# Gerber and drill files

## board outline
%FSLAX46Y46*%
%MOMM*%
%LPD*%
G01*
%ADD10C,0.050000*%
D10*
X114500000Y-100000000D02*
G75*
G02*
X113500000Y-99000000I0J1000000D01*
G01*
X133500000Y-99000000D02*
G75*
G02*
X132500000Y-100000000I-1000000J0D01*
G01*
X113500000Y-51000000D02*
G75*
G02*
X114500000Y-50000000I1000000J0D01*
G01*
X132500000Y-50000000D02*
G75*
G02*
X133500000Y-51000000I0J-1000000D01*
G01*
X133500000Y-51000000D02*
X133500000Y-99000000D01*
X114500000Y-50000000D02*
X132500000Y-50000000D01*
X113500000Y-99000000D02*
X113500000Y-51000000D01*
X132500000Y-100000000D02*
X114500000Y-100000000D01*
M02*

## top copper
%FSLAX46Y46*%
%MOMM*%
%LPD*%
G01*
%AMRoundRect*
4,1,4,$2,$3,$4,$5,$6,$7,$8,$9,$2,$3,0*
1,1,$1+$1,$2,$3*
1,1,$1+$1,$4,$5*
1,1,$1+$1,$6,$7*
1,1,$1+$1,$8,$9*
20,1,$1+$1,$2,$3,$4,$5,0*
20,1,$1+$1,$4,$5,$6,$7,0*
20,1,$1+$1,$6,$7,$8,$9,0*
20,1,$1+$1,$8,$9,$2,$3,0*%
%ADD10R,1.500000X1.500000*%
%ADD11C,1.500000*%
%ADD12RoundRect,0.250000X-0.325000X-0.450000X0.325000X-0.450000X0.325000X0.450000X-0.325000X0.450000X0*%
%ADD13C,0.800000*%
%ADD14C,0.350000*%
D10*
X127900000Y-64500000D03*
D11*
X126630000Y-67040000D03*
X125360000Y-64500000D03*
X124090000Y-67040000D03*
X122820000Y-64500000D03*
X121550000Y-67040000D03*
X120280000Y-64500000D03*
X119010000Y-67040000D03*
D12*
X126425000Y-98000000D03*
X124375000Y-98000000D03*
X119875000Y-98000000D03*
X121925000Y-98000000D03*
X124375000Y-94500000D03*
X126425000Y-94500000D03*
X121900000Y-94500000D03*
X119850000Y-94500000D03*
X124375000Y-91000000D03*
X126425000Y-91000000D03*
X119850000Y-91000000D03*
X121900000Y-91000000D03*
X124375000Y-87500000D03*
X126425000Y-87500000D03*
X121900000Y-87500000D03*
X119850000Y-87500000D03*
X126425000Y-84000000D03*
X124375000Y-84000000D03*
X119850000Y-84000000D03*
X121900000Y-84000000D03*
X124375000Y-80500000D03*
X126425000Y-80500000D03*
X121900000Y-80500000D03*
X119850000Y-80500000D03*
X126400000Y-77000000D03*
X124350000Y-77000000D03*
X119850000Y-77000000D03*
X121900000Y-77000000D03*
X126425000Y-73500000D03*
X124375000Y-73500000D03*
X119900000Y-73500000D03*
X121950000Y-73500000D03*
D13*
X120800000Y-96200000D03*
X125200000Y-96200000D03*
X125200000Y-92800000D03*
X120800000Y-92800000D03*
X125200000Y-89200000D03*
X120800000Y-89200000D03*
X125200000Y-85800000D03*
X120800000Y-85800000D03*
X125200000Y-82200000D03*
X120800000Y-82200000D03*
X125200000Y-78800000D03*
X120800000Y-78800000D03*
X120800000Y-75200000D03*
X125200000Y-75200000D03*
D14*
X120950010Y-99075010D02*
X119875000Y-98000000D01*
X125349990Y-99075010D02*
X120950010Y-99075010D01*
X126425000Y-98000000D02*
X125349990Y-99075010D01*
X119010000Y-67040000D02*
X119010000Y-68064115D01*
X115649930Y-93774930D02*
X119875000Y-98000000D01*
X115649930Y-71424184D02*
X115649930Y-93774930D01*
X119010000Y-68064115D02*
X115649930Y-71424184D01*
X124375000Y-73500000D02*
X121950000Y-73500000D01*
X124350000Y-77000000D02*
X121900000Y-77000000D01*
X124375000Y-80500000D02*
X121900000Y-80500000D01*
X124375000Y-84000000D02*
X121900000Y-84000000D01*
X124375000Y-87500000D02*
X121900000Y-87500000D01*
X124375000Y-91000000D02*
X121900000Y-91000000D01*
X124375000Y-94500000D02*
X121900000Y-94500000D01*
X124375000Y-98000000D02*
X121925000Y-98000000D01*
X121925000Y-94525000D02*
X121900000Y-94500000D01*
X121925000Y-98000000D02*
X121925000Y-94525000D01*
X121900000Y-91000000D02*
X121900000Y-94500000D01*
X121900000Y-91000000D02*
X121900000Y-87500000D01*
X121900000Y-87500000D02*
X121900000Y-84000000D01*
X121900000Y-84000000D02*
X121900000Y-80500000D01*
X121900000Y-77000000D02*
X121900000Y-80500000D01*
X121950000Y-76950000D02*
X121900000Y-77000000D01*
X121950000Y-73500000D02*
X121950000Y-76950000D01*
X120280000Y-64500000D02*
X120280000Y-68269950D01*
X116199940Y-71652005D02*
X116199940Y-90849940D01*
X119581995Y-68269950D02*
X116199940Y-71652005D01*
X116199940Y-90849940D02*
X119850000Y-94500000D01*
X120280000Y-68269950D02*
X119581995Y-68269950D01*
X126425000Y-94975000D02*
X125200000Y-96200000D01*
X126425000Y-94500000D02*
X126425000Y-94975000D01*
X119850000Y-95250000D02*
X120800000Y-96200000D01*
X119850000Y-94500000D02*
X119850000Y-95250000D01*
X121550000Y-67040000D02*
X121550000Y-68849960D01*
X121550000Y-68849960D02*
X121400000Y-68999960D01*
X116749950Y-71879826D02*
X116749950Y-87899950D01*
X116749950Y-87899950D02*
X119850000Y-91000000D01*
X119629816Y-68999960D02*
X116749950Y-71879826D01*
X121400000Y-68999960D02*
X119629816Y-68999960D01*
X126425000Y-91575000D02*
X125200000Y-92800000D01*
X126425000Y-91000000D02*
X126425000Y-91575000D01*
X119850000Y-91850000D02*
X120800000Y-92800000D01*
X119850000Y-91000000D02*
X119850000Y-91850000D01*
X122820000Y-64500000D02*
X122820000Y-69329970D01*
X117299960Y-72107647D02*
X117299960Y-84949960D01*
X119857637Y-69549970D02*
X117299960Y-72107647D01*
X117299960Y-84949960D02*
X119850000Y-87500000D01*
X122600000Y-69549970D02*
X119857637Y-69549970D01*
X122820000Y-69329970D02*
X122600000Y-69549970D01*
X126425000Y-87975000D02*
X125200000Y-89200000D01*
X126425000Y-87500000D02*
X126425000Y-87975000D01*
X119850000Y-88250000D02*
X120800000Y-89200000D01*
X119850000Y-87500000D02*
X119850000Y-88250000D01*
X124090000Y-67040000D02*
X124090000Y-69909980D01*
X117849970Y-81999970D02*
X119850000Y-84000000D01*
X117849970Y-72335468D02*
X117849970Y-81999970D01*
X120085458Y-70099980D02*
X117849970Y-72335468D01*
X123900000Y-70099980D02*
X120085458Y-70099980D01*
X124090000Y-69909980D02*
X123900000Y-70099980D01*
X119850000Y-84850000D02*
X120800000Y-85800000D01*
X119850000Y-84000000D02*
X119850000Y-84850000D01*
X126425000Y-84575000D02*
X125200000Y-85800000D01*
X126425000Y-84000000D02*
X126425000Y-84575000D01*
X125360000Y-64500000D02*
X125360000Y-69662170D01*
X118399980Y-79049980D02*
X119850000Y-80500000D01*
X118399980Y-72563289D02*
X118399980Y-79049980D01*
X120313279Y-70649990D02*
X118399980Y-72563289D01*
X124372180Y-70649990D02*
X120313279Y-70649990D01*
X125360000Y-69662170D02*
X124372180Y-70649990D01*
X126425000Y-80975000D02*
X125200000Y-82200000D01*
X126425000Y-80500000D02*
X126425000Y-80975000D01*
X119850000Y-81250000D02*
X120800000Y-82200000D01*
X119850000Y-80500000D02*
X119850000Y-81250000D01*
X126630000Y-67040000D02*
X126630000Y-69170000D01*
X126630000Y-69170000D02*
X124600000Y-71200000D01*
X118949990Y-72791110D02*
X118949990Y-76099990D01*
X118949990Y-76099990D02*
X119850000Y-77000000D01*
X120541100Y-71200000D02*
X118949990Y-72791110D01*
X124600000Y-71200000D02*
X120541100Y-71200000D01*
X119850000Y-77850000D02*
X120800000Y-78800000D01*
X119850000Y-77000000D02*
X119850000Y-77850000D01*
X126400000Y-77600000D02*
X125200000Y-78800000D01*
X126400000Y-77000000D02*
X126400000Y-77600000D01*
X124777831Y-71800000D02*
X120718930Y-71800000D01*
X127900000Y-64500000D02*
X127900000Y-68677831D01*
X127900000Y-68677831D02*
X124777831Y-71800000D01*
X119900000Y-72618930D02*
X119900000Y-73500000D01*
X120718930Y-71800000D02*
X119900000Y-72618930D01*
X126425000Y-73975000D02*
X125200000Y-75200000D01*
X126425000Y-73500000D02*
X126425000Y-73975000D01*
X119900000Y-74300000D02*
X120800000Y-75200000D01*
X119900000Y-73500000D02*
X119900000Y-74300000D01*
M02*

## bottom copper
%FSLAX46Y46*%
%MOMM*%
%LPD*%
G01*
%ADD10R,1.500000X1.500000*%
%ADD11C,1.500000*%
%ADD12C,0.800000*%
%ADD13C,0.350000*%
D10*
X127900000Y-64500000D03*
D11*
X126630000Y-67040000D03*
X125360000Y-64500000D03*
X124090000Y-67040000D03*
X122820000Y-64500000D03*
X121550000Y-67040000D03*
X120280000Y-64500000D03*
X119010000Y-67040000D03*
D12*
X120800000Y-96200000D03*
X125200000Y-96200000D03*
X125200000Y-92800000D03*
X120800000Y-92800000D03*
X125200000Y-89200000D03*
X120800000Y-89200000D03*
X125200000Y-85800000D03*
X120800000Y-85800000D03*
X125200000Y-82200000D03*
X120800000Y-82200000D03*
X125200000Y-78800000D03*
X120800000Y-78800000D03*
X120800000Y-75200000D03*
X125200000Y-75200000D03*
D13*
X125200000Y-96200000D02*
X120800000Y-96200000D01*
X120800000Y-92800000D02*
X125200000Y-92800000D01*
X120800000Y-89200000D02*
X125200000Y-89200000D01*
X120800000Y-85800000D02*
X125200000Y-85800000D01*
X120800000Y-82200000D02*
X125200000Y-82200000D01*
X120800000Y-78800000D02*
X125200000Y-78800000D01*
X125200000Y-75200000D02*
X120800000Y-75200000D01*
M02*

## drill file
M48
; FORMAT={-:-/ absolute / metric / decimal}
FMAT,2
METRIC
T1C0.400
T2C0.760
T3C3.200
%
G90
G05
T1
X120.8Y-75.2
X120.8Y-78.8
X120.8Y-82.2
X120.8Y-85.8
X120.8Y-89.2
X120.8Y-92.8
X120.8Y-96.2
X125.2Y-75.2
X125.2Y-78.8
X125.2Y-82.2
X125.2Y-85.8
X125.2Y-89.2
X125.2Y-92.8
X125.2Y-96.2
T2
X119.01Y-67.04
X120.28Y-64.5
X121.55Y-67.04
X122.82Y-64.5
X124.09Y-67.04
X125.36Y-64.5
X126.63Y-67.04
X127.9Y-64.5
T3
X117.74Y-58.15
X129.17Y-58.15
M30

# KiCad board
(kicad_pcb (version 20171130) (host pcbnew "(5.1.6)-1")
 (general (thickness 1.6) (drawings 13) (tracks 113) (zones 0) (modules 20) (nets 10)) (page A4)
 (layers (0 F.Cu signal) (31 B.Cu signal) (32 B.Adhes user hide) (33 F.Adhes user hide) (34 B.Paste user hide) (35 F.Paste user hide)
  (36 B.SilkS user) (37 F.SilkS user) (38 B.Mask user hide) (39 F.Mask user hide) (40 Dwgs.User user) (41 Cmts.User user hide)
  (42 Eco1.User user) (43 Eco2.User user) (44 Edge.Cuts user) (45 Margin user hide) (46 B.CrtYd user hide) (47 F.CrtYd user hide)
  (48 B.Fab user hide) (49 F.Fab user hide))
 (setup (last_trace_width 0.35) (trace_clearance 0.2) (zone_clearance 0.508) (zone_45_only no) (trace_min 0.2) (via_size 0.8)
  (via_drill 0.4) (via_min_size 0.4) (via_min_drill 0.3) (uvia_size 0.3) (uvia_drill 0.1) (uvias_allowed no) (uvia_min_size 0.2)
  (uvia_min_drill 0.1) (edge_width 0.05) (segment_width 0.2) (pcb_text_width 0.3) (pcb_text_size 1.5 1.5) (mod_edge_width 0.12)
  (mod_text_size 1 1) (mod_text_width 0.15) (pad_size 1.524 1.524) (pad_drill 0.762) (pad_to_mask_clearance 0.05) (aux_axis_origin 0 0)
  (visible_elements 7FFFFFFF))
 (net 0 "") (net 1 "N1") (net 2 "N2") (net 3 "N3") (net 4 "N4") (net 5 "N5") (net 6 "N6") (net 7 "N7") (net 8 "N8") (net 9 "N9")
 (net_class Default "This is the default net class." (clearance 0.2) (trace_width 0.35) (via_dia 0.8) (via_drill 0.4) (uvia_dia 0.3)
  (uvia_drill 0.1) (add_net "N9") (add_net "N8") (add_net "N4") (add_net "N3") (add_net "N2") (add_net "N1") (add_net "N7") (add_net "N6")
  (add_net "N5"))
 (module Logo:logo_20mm (layer B.Cu) (at 123.6 79.8 180)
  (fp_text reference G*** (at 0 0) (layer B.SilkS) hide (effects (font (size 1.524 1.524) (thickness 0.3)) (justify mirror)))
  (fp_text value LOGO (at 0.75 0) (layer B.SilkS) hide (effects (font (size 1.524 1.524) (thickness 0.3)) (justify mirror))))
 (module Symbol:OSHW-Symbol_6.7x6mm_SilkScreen (layer B.Cu) (at 118.1 95.9 180)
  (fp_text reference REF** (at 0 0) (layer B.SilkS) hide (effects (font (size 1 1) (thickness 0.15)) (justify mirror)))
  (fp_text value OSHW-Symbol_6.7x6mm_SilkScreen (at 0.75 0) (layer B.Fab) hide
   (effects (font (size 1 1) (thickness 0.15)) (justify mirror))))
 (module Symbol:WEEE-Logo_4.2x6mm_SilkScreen (layer B.Cu) (at 130.6 95.8 180)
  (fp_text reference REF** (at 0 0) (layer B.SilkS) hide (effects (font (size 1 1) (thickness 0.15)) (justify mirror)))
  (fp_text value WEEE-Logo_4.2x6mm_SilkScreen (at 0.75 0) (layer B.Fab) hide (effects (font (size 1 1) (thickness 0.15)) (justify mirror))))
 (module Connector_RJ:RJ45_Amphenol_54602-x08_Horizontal (layer F.Cu) (at 127.9 64.5 180)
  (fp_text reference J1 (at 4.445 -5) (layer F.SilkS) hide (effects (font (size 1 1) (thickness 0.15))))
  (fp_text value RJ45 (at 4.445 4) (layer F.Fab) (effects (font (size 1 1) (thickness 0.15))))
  (pad "" np_thru_hole circle (at 10.16 6.35 180) (size 3.2 3.2) (drill 3.2) (layers *.Cu *.Mask))
  (pad "" np_thru_hole circle (at -1.27 6.35 180) (size 3.2 3.2) (drill 3.2) (layers *.Cu *.Mask))
  (pad 1 thru_hole rect (at 0 0 180) (size 1.5 1.5) (drill 0.76) (layers *.Cu *.Mask) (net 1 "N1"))
  (pad 2 thru_hole circle (at 1.27 -2.54 180) (size 1.5 1.5) (drill 0.76) (layers *.Cu *.Mask) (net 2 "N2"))
  (pad 3 thru_hole circle (at 2.54 0 180) (size 1.5 1.5) (drill 0.76) (layers *.Cu *.Mask) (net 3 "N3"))
  (pad 4 thru_hole circle (at 3.81 -2.54 180) (size 1.5 1.5) (drill 0.76) (layers *.Cu *.Mask) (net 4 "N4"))
  (pad 5 thru_hole circle (at 5.08 0 180) (size 1.5 1.5) (drill 0.76) (layers *.Cu *.Mask) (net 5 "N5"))
  (pad 6 thru_hole circle (at 6.35 -2.54 180) (size 1.5 1.5) (drill 0.76) (layers *.Cu *.Mask) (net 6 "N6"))
  (pad 7 thru_hole circle (at 7.62 0 180) (size 1.5 1.5) (drill 0.76) (layers *.Cu *.Mask) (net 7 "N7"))
  (pad 8 thru_hole circle (at 8.89 -2.54 180) (size 1.5 1.5) (drill 0.76) (layers *.Cu *.Mask) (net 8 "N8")))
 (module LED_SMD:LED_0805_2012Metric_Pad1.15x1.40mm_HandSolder (layer F.Cu) (at 125.4 98)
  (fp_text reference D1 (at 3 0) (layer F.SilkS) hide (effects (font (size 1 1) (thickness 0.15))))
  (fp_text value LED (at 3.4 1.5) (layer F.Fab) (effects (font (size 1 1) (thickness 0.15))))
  (pad 2 smd roundrect (at 1.025 0) (size 1.15 1.4) (layers F.Cu F.Paste F.Mask) (roundrect_rratio 0.217391) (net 8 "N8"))
  (pad 1 smd roundrect (at -1.025 0) (size 1.15 1.4) (layers F.Cu F.Paste F.Mask) (roundrect_rratio 0.217391) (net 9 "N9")))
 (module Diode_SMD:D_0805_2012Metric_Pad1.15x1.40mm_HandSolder (layer F.Cu) (at 120.9 98)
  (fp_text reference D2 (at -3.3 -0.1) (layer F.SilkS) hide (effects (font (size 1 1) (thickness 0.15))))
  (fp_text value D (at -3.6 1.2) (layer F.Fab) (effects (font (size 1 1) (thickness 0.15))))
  (pad 1 smd roundrect (at -1.025 0) (size 1.15 1.4) (layers F.Cu F.Paste F.Mask) (roundrect_rratio 0.217391) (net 8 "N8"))
  (pad 2 smd roundrect (at 1.025 0) (size 1.15 1.4) (layers F.Cu F.Paste F.Mask) (roundrect_rratio 0.217391) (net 9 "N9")))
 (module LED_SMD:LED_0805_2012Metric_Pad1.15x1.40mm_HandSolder (layer F.Cu) (at 125.4 94.5)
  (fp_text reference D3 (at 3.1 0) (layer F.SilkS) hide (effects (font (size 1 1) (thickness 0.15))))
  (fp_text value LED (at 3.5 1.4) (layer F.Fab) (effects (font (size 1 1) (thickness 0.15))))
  (pad 1 smd roundrect (at -1.025 0) (size 1.15 1.4) (layers F.Cu F.Paste F.Mask) (roundrect_rratio 0.217391) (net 9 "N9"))
  (pad 2 smd roundrect (at 1.025 0) (size 1.15 1.4) (layers F.Cu F.Paste F.Mask) (roundrect_rratio 0.217391) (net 7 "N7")))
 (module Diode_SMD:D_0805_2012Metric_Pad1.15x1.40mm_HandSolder (layer F.Cu) (at 120.875 94.5)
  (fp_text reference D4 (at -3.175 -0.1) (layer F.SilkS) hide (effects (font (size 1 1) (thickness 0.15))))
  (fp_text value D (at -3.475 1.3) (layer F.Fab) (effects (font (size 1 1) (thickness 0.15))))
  (pad 2 smd roundrect (at 1.025 0) (size 1.15 1.4) (layers F.Cu F.Paste F.Mask) (roundrect_rratio 0.217391) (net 9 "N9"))
  (pad 1 smd roundrect (at -1.025 0) (size 1.15 1.4) (layers F.Cu F.Paste F.Mask) (roundrect_rratio 0.217391) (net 7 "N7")))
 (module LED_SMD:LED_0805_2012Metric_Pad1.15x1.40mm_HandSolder (layer F.Cu) (at 125.4 91)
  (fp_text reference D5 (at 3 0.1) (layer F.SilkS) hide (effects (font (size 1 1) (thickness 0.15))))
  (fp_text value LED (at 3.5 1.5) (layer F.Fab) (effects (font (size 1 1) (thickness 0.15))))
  (pad 1 smd roundrect (at -1.025 0) (size 1.15 1.4) (layers F.Cu F.Paste F.Mask) (roundrect_rratio 0.217391) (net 9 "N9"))
  (pad 2 smd roundrect (at 1.025 0) (size 1.15 1.4) (layers F.Cu F.Paste F.Mask) (roundrect_rratio 0.217391) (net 6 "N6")))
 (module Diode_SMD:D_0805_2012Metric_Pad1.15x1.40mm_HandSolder (layer F.Cu) (at 120.875 91)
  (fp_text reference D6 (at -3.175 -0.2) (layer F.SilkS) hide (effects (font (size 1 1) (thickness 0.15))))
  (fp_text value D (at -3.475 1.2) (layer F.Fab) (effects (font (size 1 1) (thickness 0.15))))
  (pad 1 smd roundrect (at -1.025 0) (size 1.15 1.4) (layers F.Cu F.Paste F.Mask) (roundrect_rratio 0.217391) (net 6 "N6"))
  (pad 2 smd roundrect (at 1.025 0) (size 1.15 1.4) (layers F.Cu F.Paste F.Mask) (roundrect_rratio 0.217391) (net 9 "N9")))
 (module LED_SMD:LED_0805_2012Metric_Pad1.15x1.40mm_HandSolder (layer F.Cu) (at 125.4 87.5)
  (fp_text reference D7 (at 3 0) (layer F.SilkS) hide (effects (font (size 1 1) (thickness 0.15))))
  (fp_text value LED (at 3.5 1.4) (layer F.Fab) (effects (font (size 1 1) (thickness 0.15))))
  (pad 1 smd roundrect (at -1.025 0) (size 1.15 1.4) (layers F.Cu F.Paste F.Mask) (roundrect_rratio 0.217391) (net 9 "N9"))
  (pad 2 smd roundrect (at 1.025 0) (size 1.15 1.4) (layers F.Cu F.Paste F.Mask) (roundrect_rratio 0.217391) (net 5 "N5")))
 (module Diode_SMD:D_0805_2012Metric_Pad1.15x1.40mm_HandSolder (layer F.Cu) (at 120.875 87.5)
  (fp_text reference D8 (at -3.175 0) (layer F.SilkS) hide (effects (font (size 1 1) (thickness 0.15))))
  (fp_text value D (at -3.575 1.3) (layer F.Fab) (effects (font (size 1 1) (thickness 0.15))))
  (pad 2 smd roundrect (at 1.025 0) (size 1.15 1.4) (layers F.Cu F.Paste F.Mask) (roundrect_rratio 0.217391) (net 9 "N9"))
  (pad 1 smd roundrect (at -1.025 0) (size 1.15 1.4) (layers F.Cu F.Paste F.Mask) (roundrect_rratio 0.217391) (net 5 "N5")))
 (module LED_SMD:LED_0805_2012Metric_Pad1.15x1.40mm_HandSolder (layer F.Cu) (at 125.4 84)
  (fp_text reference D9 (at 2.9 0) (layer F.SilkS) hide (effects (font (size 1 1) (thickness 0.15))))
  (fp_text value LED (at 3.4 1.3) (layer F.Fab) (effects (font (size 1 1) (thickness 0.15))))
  (pad 2 smd roundrect (at 1.025 0) (size 1.15 1.4) (layers F.Cu F.Paste F.Mask) (roundrect_rratio 0.217391) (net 4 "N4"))
  (pad 1 smd roundrect (at -1.025 0) (size 1.15 1.4) (layers F.Cu F.Paste F.Mask) (roundrect_rratio 0.217391) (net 9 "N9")))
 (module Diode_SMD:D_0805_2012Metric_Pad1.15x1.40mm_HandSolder (layer F.Cu) (at 120.875 84)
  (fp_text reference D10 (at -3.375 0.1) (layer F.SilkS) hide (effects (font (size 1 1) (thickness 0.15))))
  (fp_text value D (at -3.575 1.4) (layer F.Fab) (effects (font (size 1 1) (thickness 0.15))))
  (pad 1 smd roundrect (at -1.025 0) (size 1.15 1.4) (layers F.Cu F.Paste F.Mask) (roundrect_rratio 0.217391) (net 4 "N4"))
  (pad 2 smd roundrect (at 1.025 0) (size 1.15 1.4) (layers F.Cu F.Paste F.Mask) (roundrect_rratio 0.217391) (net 9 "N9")))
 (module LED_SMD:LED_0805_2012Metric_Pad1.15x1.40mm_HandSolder (layer F.Cu) (at 125.4 80.5)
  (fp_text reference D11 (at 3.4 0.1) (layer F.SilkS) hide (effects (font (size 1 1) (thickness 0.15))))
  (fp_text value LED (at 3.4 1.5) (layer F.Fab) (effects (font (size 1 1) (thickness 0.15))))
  (pad 1 smd roundrect (at -1.025 0) (size 1.15 1.4) (layers F.Cu F.Paste F.Mask) (roundrect_rratio 0.217391) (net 9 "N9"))
  (pad 2 smd roundrect (at 1.025 0) (size 1.15 1.4) (layers F.Cu F.Paste F.Mask) (roundrect_rratio 0.217391) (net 3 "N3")))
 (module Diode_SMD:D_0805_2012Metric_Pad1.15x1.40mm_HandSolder (layer F.Cu) (at 120.875 80.5)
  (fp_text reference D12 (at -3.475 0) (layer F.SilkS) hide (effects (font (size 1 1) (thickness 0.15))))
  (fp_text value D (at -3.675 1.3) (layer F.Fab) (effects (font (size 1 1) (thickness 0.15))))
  (pad 2 smd roundrect (at 1.025 0) (size 1.15 1.4) (layers F.Cu F.Paste F.Mask) (roundrect_rratio 0.217391) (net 9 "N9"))
  (pad 1 smd roundrect (at -1.025 0) (size 1.15 1.4) (layers F.Cu F.Paste F.Mask) (roundrect_rratio 0.217391) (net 3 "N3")))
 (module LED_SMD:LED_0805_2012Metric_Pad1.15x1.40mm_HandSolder (layer F.Cu) (at 125.375 77)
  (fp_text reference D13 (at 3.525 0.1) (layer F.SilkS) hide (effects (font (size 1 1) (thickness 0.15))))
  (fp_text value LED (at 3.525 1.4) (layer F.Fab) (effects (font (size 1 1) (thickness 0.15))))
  (pad 2 smd roundrect (at 1.025 0) (size 1.15 1.4) (layers F.Cu F.Paste F.Mask) (roundrect_rratio 0.217391) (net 2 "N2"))
  (pad 1 smd roundrect (at -1.025 0) (size 1.15 1.4) (layers F.Cu F.Paste F.Mask) (roundrect_rratio 0.217391) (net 9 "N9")))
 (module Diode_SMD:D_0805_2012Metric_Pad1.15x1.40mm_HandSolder (layer F.Cu) (at 120.875 77)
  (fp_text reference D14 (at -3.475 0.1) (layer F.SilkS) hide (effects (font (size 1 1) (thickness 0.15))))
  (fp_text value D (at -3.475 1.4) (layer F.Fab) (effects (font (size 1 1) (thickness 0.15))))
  (pad 1 smd roundrect (at -1.025 0) (size 1.15 1.4) (layers F.Cu F.Paste F.Mask) (roundrect_rratio 0.217391) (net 2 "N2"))
  (pad 2 smd roundrect (at 1.025 0) (size 1.15 1.4) (layers F.Cu F.Paste F.Mask) (roundrect_rratio 0.217391) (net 9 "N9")))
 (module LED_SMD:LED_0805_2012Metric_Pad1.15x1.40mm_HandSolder (layer F.Cu) (at 125.4 73.5)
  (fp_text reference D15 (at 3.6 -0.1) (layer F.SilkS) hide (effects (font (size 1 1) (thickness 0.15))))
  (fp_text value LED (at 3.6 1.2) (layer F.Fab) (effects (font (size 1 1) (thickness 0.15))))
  (pad 2 smd roundrect (at 1.025 0) (size 1.15 1.4) (layers F.Cu F.Paste F.Mask) (roundrect_rratio 0.217391) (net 1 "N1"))
  (pad 1 smd roundrect (at -1.025 0) (size 1.15 1.4) (layers F.Cu F.Paste F.Mask) (roundrect_rratio 0.217391) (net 9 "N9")))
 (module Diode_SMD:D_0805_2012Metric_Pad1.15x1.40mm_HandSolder (layer F.Cu) (at 120.925 73.5)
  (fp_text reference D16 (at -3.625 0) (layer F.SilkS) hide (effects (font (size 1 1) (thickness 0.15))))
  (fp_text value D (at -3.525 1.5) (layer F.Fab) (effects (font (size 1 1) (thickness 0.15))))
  (pad 1 smd roundrect (at -1.025 0) (size 1.15 1.4) (layers F.Cu F.Paste F.Mask) (roundrect_rratio 0.217391) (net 1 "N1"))
  (pad 2 smd roundrect (at 1.025 0) (size 1.15 1.4) (layers F.Cu F.Paste F.Mask) (roundrect_rratio 0.217391) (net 9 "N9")))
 (gr_arc (start 114.5 99) (end 113.5 99) (angle -90) (layer Edge.Cuts) (width 0.05))
 (gr_arc (start 132.5 99) (end 132.5 100) (angle -90) (layer Edge.Cuts) (width 0.05))
 (gr_arc (start 114.5 51) (end 114.5 50) (angle -90) (layer Edge.Cuts) (width 0.05))
 (gr_arc (start 132.5 51) (end 133.5 51) (angle -90) (layer Edge.Cuts) (width 0.05))
 (gr_line (start 133.5 51) (end 133.5 99) (layer Edge.Cuts) (width 0.05))
 (gr_line (start 114.5 50) (end 132.5 50) (layer Edge.Cuts) (width 0.05))
 (gr_line (start 113.5 99) (end 113.5 51) (layer Edge.Cuts) (width 0.05))
 (gr_line (start 132.5 100) (end 114.5 100) (layer Edge.Cuts) (width 0.05))
 (segment (start 120.95001 99.07501) (end 119.875 98) (width 0.35) (layer F.Cu) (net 8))
 (segment (start 125.34999 99.07501) (end 120.95001 99.07501) (width 0.35) (layer F.Cu) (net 8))
 (segment (start 126.425 98) (end 125.34999 99.07501) (width 0.35) (layer F.Cu) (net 8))
 (segment (start 119.01 67.04) (end 119.01 68.064115) (width 0.35) (layer F.Cu) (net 8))
 (segment (start 115.64993 93.77493) (end 119.875 98) (width 0.35) (layer F.Cu) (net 8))
 (segment (start 115.64993 71.424184) (end 115.64993 93.77493) (width 0.35) (layer F.Cu) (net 8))
 (segment (start 119.01 68.064115) (end 115.64993 71.424184) (width 0.35) (layer F.Cu) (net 8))
 (segment (start 124.375 73.5) (end 121.95 73.5) (width 0.35) (layer F.Cu) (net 9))
 (segment (start 124.35 77) (end 121.9 77) (width 0.35) (layer F.Cu) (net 9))
 (segment (start 124.375 80.5) (end 121.9 80.5) (width 0.35) (layer F.Cu) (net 9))
 (segment (start 124.375 84) (end 121.9 84) (width 0.35) (layer F.Cu) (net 9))
 (segment (start 124.375 87.5) (end 121.9 87.5) (width 0.35) (layer F.Cu) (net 9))
 (segment (start 124.375 91) (end 121.9 91) (width 0.35) (layer F.Cu) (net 9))
 (segment (start 124.375 94.5) (end 121.9 94.5) (width 0.35) (layer F.Cu) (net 9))
 (segment (start 124.375 98) (end 121.925 98) (width 0.35) (layer F.Cu) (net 9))
 (segment (start 121.925 94.525) (end 121.9 94.5) (width 0.35) (layer F.Cu) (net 9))
 (segment (start 121.925 98) (end 121.925 94.525) (width 0.35) (layer F.Cu) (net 9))
 (segment (start 121.9 91) (end 121.9 94.5) (width 0.35) (layer F.Cu) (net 9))
 (segment (start 121.9 91) (end 121.9 87.5) (width 0.35) (layer F.Cu) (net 9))
 (segment (start 121.9 87.5) (end 121.9 84) (width 0.35) (layer F.Cu) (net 9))
 (segment (start 121.9 84) (end 121.9 80.5) (width 0.35) (layer F.Cu) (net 9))
 (segment (start 121.9 77) (end 121.9 80.5) (width 0.35) (layer F.Cu) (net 9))
 (segment (start 121.95 76.95) (end 121.9 77) (width 0.35) (layer F.Cu) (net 9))
 (segment (start 121.95 73.5) (end 121.95 76.95) (width 0.35) (layer F.Cu) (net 9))
 (via (at 120.8 96.2) (size 0.8) (drill 0.4) (layers F.Cu B.Cu) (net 7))
 (via (at 125.2 96.2) (size 0.8) (drill 0.4) (layers F.Cu B.Cu) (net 7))
 (segment (start 120.28 64.5) (end 120.28 68.26995) (width 0.35) (layer F.Cu) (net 7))
 (segment (start 116.19994 71.652005) (end 116.19994 90.84994) (width 0.35) (layer F.Cu) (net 7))
 (segment (start 119.581995 68.26995) (end 116.19994 71.652005) (width 0.35) (layer F.Cu) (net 7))
 (segment (start 116.19994 90.84994) (end 119.85 94.5) (width 0.35) (layer F.Cu) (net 7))
 (segment (start 120.28 68.26995) (end 119.581995 68.26995) (width 0.35) (layer F.Cu) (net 7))
 (segment (start 125.2 96.2) (end 120.8 96.2) (width 0.35) (layer B.Cu) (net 7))
 (segment (start 126.425 94.975) (end 125.2 96.2) (width 0.35) (layer F.Cu) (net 7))
 (segment (start 126.425 94.5) (end 126.425 94.975) (width 0.35) (layer F.Cu) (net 7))
 (segment (start 119.85 95.25) (end 120.8 96.2) (width 0.35) (layer F.Cu) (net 7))
 (segment (start 119.85 94.5) (end 119.85 95.25) (width 0.35) (layer F.Cu) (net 7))
 (via (at 125.2 92.8) (size 0.8) (drill 0.4) (layers F.Cu B.Cu) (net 6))
 (via (at 120.8 92.8) (size 0.8) (drill 0.4) (layers F.Cu B.Cu) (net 6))
 (segment (start 121.55 67.04) (end 121.55 68.84996) (width 0.35) (layer F.Cu) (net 6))
 (segment (start 121.55 68.84996) (end 121.4 68.99996) (width 0.35) (layer F.Cu) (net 6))
 (segment (start 116.74995 71.879826) (end 116.74995 87.89995) (width 0.35) (layer F.Cu) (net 6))
 (segment (start 116.74995 87.89995) (end 119.85 91) (width 0.35) (layer F.Cu) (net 6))
 (segment (start 119.629816 68.99996) (end 116.74995 71.879826) (width 0.35) (layer F.Cu) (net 6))
 (segment (start 121.4 68.99996) (end 119.629816 68.99996) (width 0.35) (layer F.Cu) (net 6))
 (segment (start 120.8 92.8) (end 125.2 92.8) (width 0.35) (layer B.Cu) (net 6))
 (segment (start 126.425 91.575) (end 125.2 92.8) (width 0.35) (layer F.Cu) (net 6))
 (segment (start 126.425 91) (end 126.425 91.575) (width 0.35) (layer F.Cu) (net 6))
 (segment (start 119.85 91.85) (end 120.8 92.8) (width 0.35) (layer F.Cu) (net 6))
 (segment (start 119.85 91) (end 119.85 91.85) (width 0.35) (layer F.Cu) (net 6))
 (via (at 125.2 89.2) (size 0.8) (drill 0.4) (layers F.Cu B.Cu) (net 5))
 (via (at 120.8 89.2) (size 0.8) (drill 0.4) (layers F.Cu B.Cu) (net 5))
 (segment (start 122.82 64.5) (end 122.82 69.32997) (width 0.35) (layer F.Cu) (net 5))
 (segment (start 117.29996 72.107647) (end 117.29996 84.94996) (width 0.35) (layer F.Cu) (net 5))
 (segment (start 119.857637 69.54997) (end 117.29996 72.107647) (width 0.35) (layer F.Cu) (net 5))
 (segment (start 117.29996 84.94996) (end 119.85 87.5) (width 0.35) (layer F.Cu) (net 5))
 (segment (start 122.6 69.54997) (end 119.857637 69.54997) (width 0.35) (layer F.Cu) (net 5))
 (segment (start 122.82 69.32997) (end 122.6 69.54997) (width 0.35) (layer F.Cu) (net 5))
 (segment (start 120.8 89.2) (end 125.2 89.2) (width 0.35) (layer B.Cu) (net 5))
 (segment (start 126.425 87.975) (end 125.2 89.2) (width 0.35) (layer F.Cu) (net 5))
 (segment (start 126.425 87.5) (end 126.425 87.975) (width 0.35) (layer F.Cu) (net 5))
 (segment (start 119.85 88.25) (end 120.8 89.2) (width 0.35) (layer F.Cu) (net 5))
 (segment (start 119.85 87.5) (end 119.85 88.25) (width 0.35) (layer F.Cu) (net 5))
 (via (at 125.2 85.8) (size 0.8) (drill 0.4) (layers F.Cu B.Cu) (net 4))
 (via (at 120.8 85.8) (size 0.8) (drill 0.4) (layers F.Cu B.Cu) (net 4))
 (segment (start 124.09 67.04) (end 124.09 69.90998) (width 0.35) (layer F.Cu) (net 4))
 (segment (start 117.84997 81.99997) (end 119.85 84) (width 0.35) (layer F.Cu) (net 4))
 (segment (start 117.84997 72.335468) (end 117.84997 81.99997) (width 0.35) (layer F.Cu) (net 4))
 (segment (start 120.085458 70.09998) (end 117.84997 72.335468) (width 0.35) (layer F.Cu) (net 4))
 (segment (start 123.9 70.09998) (end 120.085458 70.09998) (width 0.35) (layer F.Cu) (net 4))
 (segment (start 124.09 69.90998) (end 123.9 70.09998) (width 0.35) (layer F.Cu) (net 4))
 (segment (start 120.8 85.8) (end 125.2 85.8) (width 0.35) (layer B.Cu) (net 4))
 (segment (start 119.85 84.85) (end 120.8 85.8) (width 0.35) (layer F.Cu) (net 4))
 (segment (start 119.85 84) (end 119.85 84.85) (width 0.35) (layer F.Cu) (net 4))
 (segment (start 126.425 84.575) (end 125.2 85.8) (width 0.35) (layer F.Cu) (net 4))
 (segment (start 126.425 84) (end 126.425 84.575) (width 0.35) (layer F.Cu) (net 4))
 (via (at 125.2 82.2) (size 0.8) (drill 0.4) (layers F.Cu B.Cu) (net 3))
 (via (at 120.8 82.2) (size 0.8) (drill 0.4) (layers F.Cu B.Cu) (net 3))
 (segment (start 125.36 64.5) (end 125.36 69.66217) (width 0.35) (layer F.Cu) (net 3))
 (segment (start 118.39998 79.04998) (end 119.85 80.5) (width 0.35) (layer F.Cu) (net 3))
 (segment (start 118.39998 72.563289) (end 118.39998 79.04998) (width 0.35) (layer F.Cu) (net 3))
 (segment (start 120.313279 70.64999) (end 118.39998 72.563289) (width 0.35) (layer F.Cu) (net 3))
 (segment (start 124.37218 70.64999) (end 120.313279 70.64999) (width 0.35) (layer F.Cu) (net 3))
 (segment (start 125.36 69.66217) (end 124.37218 70.64999) (width 0.35) (layer F.Cu) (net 3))
 (segment (start 120.8 82.2) (end 125.2 82.2) (width 0.35) (layer B.Cu) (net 3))
 (segment (start 126.425 80.975) (end 125.2 82.2) (width 0.35) (layer F.Cu) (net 3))
 (segment (start 126.425 80.5) (end 126.425 80.975) (width 0.35) (layer F.Cu) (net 3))
 (segment (start 119.85 81.25) (end 120.8 82.2) (width 0.35) (layer F.Cu) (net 3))
 (segment (start 119.85 80.5) (end 119.85 81.25) (width 0.35) (layer F.Cu) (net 3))
 (via (at 125.2 78.8) (size 0.8) (drill 0.4) (layers F.Cu B.Cu) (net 2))
 (via (at 120.8 78.8) (size 0.8) (drill 0.4) (layers F.Cu B.Cu) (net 2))
 (segment (start 126.63 67.04) (end 126.63 69.17) (width 0.35) (layer F.Cu) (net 2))
 (segment (start 126.63 69.17) (end 124.6 71.2) (width 0.35) (layer F.Cu) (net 2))
 (segment (start 118.94999 72.79111) (end 118.94999 76.09999) (width 0.35) (layer F.Cu) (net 2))
 (segment (start 118.94999 76.09999) (end 119.85 77) (width 0.35) (layer F.Cu) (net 2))
 (segment (start 120.5411 71.2) (end 118.94999 72.79111) (width 0.35) (layer F.Cu) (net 2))
 (segment (start 124.6 71.2) (end 120.5411 71.2) (width 0.35) (layer F.Cu) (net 2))
 (segment (start 120.8 78.8) (end 125.2 78.8) (width 0.35) (layer B.Cu) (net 2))
 (segment (start 119.85 77.85) (end 120.8 78.8) (width 0.35) (layer F.Cu) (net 2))
 (segment (start 119.85 77) (end 119.85 77.85) (width 0.35) (layer F.Cu) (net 2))
 (segment (start 126.4 77.6) (end 125.2 78.8) (width 0.35) (layer F.Cu) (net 2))
 (segment (start 126.4 77) (end 126.4 77.6) (width 0.35) (layer F.Cu) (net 2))
 (via (at 120.8 75.2) (size 0.8) (drill 0.4) (layers F.Cu B.Cu) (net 1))
 (via (at 125.2 75.2) (size 0.8) (drill 0.4) (layers F.Cu B.Cu) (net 1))
 (segment (start 124.777831 71.8) (end 120.71893 71.8) (width 0.35) (layer F.Cu) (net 1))
 (segment (start 127.9 64.5) (end 127.9 68.677831) (width 0.35) (layer F.Cu) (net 1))
 (segment (start 127.9 68.677831) (end 124.777831 71.8) (width 0.35) (layer F.Cu) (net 1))
 (segment (start 119.9 72.61893) (end 119.9 73.5) (width 0.35) (layer F.Cu) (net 1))
 (segment (start 120.71893 71.8) (end 119.9 72.61893) (width 0.35) (layer F.Cu) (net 1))
 (segment (start 125.2 75.2) (end 120.8 75.2) (width 0.35) (layer B.Cu) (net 1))
 (segment (start 126.425 73.975) (end 125.2 75.2) (width 0.35) (layer F.Cu) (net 1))
 (segment (start 126.425 73.5) (end 126.425 73.975) (width 0.35) (layer F.Cu) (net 1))
 (segment (start 119.9 74.3) (end 120.8 75.2) (width 0.35) (layer F.Cu) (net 1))
 (segment (start 119.9 73.5) (end 119.9 74.3) (width 0.35) (layer F.Cu) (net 1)))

